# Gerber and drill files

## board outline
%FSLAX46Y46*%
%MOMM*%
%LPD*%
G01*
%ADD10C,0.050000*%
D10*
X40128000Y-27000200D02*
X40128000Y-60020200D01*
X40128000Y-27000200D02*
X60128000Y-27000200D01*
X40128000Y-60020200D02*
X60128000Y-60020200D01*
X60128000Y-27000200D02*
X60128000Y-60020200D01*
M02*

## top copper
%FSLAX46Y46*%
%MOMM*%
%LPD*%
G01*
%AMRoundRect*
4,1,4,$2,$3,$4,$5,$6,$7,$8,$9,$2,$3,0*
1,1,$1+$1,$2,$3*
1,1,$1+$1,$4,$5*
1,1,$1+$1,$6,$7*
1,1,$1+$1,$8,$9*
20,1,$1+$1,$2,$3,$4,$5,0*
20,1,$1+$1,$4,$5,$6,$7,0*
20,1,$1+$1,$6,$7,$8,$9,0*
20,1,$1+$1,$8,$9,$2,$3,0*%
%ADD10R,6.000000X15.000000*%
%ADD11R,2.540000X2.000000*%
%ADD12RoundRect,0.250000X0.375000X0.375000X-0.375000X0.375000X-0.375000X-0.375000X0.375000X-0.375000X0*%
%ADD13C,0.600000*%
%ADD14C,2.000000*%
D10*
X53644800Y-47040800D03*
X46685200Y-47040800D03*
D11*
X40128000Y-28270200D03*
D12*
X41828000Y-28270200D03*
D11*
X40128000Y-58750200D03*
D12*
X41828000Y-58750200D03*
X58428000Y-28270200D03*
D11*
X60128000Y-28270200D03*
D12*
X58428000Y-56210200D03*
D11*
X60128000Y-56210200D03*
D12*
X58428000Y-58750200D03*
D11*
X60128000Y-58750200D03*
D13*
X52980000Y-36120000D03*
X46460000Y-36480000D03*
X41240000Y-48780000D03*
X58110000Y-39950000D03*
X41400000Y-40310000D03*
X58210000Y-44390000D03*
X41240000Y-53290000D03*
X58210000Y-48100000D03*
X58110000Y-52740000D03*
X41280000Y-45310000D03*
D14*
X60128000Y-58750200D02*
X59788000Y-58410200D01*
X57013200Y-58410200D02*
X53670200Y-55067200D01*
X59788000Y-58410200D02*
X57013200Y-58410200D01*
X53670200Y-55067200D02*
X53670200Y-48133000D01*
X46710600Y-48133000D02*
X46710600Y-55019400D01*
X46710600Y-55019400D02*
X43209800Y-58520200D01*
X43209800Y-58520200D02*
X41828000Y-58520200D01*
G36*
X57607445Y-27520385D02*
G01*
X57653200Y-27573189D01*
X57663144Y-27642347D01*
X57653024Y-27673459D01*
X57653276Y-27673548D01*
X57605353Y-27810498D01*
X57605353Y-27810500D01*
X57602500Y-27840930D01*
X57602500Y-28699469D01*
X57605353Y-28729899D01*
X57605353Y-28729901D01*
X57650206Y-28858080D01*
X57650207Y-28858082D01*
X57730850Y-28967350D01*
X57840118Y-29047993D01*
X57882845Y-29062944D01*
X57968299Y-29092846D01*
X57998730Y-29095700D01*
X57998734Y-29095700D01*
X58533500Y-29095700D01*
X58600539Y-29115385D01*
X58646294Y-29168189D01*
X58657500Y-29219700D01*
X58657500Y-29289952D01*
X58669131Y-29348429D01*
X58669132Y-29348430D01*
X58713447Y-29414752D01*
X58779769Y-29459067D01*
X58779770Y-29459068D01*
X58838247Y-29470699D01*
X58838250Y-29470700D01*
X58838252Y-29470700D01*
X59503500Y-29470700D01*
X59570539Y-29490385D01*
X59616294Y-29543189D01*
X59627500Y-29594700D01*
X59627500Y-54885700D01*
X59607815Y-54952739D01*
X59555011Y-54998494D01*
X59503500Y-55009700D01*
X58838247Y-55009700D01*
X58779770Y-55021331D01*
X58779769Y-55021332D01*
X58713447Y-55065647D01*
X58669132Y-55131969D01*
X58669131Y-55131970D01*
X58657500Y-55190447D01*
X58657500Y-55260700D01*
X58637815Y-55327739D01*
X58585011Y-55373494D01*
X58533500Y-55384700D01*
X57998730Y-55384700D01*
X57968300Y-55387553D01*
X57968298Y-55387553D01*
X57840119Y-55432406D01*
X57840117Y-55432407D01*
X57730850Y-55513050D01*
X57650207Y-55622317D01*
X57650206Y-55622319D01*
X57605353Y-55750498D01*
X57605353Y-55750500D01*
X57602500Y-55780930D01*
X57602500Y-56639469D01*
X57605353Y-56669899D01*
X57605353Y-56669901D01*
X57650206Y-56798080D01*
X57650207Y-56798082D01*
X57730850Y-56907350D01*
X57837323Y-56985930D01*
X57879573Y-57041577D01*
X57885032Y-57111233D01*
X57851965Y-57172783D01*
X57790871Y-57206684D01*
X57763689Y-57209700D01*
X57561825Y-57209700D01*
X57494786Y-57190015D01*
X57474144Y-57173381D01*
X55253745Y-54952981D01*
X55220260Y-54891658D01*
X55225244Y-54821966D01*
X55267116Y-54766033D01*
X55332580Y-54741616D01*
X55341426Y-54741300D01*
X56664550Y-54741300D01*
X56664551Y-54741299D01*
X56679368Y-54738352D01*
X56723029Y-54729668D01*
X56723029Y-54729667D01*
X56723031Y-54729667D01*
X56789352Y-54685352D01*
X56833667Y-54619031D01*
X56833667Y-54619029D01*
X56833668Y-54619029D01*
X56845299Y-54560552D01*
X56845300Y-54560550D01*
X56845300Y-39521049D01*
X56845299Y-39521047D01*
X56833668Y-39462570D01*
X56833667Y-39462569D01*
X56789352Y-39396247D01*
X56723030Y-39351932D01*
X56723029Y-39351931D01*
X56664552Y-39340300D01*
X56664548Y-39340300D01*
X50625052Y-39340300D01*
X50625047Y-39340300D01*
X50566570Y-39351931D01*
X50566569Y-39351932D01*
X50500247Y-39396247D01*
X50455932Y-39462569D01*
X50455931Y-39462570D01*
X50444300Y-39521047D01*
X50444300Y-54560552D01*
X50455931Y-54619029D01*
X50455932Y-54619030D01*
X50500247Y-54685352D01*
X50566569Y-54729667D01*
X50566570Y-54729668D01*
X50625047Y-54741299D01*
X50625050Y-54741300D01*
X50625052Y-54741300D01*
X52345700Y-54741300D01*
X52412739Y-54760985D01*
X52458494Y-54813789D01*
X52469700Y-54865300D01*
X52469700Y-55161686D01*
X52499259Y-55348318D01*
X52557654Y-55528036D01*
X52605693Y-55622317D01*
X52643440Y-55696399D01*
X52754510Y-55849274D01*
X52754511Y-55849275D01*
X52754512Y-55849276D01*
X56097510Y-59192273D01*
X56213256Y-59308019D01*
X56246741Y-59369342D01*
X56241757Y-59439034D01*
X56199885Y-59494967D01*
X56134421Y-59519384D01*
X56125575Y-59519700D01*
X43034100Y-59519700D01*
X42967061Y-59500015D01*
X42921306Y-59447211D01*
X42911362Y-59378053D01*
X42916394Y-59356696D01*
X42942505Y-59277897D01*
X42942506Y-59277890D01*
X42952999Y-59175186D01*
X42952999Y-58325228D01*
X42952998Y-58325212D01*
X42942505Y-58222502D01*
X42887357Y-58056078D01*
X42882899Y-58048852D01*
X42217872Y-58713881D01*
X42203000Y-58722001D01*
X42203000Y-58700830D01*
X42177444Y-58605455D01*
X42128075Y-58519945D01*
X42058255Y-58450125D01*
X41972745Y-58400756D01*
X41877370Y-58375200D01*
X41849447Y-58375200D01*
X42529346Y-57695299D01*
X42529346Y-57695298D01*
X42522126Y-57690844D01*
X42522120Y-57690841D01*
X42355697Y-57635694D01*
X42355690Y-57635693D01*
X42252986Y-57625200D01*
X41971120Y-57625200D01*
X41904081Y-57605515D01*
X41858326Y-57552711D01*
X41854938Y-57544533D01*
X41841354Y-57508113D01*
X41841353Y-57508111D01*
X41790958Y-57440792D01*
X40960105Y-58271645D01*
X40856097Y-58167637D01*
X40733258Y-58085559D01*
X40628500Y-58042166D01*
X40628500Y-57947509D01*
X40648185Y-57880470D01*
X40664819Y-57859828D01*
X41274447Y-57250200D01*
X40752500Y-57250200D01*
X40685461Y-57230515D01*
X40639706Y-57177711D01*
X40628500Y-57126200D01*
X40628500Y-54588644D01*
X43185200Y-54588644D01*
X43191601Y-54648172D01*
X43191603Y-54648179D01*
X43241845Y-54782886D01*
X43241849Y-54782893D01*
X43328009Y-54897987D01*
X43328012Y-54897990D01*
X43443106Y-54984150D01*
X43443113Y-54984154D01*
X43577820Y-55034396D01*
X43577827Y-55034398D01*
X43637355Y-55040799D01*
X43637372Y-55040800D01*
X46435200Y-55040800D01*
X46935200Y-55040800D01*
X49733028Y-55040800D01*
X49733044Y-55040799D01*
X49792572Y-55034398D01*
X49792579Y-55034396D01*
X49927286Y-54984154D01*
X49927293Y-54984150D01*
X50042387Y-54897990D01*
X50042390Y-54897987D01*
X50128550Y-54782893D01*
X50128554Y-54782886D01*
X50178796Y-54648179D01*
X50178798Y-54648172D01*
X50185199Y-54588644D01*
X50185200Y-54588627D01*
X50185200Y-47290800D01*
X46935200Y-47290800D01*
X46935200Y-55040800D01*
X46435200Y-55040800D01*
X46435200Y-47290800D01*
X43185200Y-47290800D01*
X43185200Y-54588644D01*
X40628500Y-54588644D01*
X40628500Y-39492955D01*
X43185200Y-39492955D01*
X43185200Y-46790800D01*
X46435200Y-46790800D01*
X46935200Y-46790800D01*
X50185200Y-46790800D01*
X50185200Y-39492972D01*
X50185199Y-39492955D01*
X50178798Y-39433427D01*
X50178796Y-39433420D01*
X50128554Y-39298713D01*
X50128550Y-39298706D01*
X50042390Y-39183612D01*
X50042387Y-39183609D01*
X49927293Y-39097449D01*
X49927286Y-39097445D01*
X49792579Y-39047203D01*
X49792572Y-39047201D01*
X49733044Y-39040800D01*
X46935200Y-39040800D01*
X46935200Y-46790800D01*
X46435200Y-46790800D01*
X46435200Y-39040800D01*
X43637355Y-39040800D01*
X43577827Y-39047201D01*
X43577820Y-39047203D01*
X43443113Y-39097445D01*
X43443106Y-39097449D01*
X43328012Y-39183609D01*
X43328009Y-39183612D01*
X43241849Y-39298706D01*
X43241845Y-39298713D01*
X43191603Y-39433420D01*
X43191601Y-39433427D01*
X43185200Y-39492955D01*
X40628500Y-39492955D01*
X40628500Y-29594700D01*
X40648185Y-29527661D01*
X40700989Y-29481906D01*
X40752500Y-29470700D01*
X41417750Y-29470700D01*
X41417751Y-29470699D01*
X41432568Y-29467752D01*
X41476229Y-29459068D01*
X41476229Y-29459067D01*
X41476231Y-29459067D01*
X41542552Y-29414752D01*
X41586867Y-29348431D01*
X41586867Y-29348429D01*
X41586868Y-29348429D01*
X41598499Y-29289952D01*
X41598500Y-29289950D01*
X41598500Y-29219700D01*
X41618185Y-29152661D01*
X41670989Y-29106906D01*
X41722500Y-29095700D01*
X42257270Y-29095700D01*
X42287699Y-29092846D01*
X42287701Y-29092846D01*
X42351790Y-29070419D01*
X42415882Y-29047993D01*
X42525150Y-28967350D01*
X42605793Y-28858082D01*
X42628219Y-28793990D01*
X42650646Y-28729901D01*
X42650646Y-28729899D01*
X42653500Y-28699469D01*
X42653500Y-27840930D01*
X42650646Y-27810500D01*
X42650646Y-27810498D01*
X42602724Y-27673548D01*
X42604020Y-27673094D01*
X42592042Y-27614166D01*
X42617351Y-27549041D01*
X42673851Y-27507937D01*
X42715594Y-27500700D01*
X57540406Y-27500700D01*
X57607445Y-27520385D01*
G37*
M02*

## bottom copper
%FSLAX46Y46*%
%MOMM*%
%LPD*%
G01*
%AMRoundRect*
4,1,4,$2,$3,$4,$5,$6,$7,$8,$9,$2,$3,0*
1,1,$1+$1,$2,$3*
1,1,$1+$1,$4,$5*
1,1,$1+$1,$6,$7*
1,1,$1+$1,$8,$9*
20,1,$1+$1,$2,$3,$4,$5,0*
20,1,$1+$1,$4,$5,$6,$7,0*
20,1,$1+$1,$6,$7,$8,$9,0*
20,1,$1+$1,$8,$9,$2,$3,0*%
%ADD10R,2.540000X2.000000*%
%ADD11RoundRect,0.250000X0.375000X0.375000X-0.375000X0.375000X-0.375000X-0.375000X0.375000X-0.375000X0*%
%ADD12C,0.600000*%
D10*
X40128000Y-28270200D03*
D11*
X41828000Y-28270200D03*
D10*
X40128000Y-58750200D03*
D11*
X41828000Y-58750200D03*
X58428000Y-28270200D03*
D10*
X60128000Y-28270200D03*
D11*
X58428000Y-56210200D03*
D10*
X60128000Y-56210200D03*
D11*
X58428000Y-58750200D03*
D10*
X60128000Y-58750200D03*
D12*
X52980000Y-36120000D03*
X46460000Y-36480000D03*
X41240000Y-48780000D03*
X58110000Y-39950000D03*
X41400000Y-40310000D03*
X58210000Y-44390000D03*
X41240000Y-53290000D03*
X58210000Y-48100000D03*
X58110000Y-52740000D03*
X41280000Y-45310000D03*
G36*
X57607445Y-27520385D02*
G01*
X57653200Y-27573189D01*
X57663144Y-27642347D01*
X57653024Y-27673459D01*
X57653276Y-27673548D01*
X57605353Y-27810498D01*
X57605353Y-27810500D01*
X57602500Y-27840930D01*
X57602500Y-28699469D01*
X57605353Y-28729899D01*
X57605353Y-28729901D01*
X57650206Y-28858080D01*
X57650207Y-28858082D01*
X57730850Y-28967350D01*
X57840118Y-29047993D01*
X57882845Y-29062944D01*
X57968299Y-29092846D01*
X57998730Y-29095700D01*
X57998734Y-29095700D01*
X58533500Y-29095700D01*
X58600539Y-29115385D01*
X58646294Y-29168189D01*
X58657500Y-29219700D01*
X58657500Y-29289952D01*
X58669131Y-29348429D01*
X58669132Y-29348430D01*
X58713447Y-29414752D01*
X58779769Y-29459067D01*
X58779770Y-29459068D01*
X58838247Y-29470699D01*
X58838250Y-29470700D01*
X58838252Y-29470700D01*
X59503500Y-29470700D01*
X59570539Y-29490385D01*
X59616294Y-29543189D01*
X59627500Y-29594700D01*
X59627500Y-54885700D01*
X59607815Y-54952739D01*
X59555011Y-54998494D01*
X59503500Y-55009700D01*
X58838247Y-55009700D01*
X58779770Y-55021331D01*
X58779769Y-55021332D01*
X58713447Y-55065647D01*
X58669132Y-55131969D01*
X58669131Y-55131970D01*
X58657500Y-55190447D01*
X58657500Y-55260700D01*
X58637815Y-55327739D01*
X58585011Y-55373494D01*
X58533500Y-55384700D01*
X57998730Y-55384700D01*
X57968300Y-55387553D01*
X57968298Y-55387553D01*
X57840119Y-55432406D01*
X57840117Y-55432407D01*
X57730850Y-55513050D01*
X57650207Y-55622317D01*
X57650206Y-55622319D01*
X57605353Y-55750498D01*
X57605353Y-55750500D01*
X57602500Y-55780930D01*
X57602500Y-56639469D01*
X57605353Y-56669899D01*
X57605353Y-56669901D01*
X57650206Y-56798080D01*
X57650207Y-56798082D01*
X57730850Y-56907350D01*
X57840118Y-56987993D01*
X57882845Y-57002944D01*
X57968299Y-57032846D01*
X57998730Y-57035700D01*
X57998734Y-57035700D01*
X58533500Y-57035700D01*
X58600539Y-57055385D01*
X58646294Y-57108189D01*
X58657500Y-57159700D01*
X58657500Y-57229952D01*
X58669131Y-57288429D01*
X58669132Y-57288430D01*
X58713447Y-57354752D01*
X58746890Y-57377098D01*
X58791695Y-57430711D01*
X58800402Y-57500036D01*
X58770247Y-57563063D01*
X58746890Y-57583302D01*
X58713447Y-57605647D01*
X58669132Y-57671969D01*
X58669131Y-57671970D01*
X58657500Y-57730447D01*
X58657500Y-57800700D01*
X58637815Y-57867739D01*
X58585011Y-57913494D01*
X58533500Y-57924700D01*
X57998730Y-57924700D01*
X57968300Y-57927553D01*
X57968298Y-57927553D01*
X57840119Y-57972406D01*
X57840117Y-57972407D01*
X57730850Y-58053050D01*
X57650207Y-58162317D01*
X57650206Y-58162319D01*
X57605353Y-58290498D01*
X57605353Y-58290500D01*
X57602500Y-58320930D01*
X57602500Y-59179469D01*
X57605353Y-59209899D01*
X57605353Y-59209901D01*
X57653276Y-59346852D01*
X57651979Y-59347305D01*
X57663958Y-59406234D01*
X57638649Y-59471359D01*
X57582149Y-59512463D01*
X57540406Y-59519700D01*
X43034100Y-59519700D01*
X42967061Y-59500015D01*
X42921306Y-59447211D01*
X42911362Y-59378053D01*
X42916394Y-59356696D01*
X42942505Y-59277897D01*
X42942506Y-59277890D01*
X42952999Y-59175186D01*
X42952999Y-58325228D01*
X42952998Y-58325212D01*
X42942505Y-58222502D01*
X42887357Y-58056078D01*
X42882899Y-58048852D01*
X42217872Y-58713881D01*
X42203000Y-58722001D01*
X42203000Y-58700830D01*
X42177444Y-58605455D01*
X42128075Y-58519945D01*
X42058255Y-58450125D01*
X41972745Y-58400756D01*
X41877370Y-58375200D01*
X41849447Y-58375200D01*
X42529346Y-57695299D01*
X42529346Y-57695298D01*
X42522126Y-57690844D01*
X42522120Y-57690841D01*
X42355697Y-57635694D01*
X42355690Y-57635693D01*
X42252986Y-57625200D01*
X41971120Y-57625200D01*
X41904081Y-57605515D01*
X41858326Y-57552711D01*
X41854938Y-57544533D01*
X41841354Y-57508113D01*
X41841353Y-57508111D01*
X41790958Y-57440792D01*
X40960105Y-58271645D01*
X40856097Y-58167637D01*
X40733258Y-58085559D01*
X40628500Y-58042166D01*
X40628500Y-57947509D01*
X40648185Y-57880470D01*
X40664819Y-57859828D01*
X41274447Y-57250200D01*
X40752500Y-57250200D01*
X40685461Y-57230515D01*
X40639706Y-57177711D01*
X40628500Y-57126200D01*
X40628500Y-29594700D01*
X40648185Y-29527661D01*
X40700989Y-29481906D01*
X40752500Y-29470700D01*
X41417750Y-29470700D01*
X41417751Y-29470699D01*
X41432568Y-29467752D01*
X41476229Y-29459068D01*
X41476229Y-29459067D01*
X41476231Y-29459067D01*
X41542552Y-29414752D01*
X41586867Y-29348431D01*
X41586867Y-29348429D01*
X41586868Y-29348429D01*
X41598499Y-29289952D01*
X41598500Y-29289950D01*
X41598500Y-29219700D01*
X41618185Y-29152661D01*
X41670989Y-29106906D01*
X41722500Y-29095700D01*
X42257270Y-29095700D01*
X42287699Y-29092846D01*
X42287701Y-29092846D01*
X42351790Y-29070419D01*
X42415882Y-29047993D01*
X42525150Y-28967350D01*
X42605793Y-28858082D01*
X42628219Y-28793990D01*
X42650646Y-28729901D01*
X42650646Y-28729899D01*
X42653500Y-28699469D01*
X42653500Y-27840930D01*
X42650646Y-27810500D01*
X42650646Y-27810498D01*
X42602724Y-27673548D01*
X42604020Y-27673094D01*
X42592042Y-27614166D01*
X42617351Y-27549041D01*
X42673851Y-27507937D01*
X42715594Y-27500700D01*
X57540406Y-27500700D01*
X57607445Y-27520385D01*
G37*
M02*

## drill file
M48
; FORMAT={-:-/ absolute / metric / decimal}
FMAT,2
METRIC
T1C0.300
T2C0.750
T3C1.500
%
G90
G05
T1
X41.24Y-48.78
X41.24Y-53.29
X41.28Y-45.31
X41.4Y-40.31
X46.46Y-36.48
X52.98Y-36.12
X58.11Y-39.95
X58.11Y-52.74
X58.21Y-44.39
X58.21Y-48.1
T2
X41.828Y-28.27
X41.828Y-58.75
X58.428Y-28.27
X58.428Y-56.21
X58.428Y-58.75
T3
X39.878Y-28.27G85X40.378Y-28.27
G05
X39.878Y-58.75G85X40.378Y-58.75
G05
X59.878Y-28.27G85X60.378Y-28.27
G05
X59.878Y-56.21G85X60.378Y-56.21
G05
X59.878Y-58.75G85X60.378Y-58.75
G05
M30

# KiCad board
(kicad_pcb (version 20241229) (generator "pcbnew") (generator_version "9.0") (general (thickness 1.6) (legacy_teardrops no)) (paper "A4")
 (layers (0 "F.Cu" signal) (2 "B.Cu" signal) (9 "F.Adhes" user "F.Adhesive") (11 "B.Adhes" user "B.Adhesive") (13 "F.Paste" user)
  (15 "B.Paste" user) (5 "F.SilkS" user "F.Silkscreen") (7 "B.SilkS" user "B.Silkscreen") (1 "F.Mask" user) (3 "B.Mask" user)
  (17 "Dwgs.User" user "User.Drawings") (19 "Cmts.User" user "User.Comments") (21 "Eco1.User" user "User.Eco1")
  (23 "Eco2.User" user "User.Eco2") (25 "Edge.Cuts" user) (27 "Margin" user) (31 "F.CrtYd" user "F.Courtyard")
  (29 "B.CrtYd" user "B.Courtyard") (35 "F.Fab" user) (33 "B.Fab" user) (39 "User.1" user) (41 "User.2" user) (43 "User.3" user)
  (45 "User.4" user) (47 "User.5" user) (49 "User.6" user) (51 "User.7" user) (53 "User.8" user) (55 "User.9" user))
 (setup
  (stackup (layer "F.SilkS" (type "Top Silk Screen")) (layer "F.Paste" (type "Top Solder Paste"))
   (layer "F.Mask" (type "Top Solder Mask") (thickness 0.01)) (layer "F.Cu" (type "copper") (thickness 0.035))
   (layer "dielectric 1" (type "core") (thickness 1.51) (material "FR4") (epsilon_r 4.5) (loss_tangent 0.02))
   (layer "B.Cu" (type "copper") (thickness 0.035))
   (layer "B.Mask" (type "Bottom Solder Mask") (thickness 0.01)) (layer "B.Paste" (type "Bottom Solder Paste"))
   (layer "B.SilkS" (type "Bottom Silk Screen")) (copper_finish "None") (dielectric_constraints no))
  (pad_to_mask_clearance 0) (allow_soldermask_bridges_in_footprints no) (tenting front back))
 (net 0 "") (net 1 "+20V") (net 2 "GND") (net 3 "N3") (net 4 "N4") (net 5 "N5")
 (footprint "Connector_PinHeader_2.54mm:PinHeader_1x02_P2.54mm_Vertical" (layer "F.Cu") (at 51.181 40.7924 -90)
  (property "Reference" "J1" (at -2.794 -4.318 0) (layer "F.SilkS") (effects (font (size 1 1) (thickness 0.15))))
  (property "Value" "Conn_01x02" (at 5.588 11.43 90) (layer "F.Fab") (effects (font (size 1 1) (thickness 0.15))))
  (pad "1" smd rect (at 6.2484 -2.4638) (size 6 15) (layers "F.Cu" "F.Mask" "F.Paste") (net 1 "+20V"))
  (pad "2" smd rect (at 6.2484 4.4958) (size 6 15) (layers "F.Cu" "F.Mask" "F.Paste") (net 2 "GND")))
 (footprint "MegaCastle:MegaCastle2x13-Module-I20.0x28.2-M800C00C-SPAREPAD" (layer "F.Cu") (at 50.128 43.5102)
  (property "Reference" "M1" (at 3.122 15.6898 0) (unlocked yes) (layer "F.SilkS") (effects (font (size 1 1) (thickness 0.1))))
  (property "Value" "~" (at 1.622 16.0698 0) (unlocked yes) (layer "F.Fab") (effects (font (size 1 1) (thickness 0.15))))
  (fp_line (start -10 -16.51) (end -10 16.51) (stroke (width 0.05) (type default)) (layer "Edge.Cuts"))
  (fp_line (start -10 -16.51) (end 10 -16.51) (stroke (width 0.05) (type default)) (layer "Edge.Cuts"))
  (fp_line (start -10 16.51) (end 10 16.51) (stroke (width 0.05) (type default)) (layer "Edge.Cuts"))
  (fp_line (start 10 -16.51) (end 10 16.51) (stroke (width 0.05) (type default)) (layer "Edge.Cuts"))
  (pad "1" thru_hole rect (at -10 -15.24) (size 2.54 2) (drill oval 2 1.5) (layers "*.Cu" "*.Mask") (remove_unused_layers no) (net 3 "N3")
   (thermal_bridge_angle 45))
  (pad "1" thru_hole roundrect (at -8.3 -15.24 180) (size 1.25 1.25) (drill 0.75) (layers "*.Cu" "*.Mask") (remove_unused_layers no)
   (roundrect_rratio 0.2) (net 3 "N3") (thermal_bridge_angle 45))
  (pad "13" thru_hole rect (at -10 15.24) (size 2.54 2) (drill oval 2 1.5) (layers "*.Cu" "*.Mask") (remove_unused_layers no) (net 2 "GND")
   (thermal_bridge_angle 45))
  (pad "13" thru_hole roundrect (at -8.3 15.24 180) (size 1.25 1.25) (drill 0.75) (layers "*.Cu" "*.Mask") (remove_unused_layers no)
   (roundrect_rratio 0.2) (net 2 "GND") (thermal_bridge_angle 45))
  (pad "14" thru_hole roundrect (at 8.3 -15.24 180) (size 1.25 1.25) (drill 0.75) (layers "*.Cu" "*.Mask") (remove_unused_layers no)
   (roundrect_rratio 0.2) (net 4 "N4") (thermal_bridge_angle 45))
  (pad "14" thru_hole rect (at 10 -15.24) (size 2.54 2) (drill oval 2 1.5) (layers "*.Cu" "*.Mask") (remove_unused_layers no) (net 4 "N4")
   (thermal_bridge_angle 45))
  (pad "25" thru_hole roundrect (at 8.3 12.7 180) (size 1.25 1.25) (drill 0.75) (layers "*.Cu" "*.Mask") (remove_unused_layers no)
   (roundrect_rratio 0.2) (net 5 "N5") (thermal_bridge_angle 45))
  (pad "25" thru_hole rect (at 10 12.7) (size 2.54 2) (drill oval 2 1.5) (layers "*.Cu" "*.Mask") (remove_unused_layers no) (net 5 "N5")
   (thermal_bridge_angle 45))
  (pad "26" thru_hole roundrect (at 8.3 15.24 180) (size 1.25 1.25) (drill 0.75) (layers "*.Cu" "*.Mask") (remove_unused_layers no)
   (roundrect_rratio 0.2) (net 1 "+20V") (thermal_bridge_angle 45))
  (pad "26" thru_hole rect (at 10 15.24) (size 2.54 2) (drill oval 2 1.5) (layers "*.Cu" "*.Mask") (remove_unused_layers no) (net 1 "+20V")
   (thermal_bridge_angle 45))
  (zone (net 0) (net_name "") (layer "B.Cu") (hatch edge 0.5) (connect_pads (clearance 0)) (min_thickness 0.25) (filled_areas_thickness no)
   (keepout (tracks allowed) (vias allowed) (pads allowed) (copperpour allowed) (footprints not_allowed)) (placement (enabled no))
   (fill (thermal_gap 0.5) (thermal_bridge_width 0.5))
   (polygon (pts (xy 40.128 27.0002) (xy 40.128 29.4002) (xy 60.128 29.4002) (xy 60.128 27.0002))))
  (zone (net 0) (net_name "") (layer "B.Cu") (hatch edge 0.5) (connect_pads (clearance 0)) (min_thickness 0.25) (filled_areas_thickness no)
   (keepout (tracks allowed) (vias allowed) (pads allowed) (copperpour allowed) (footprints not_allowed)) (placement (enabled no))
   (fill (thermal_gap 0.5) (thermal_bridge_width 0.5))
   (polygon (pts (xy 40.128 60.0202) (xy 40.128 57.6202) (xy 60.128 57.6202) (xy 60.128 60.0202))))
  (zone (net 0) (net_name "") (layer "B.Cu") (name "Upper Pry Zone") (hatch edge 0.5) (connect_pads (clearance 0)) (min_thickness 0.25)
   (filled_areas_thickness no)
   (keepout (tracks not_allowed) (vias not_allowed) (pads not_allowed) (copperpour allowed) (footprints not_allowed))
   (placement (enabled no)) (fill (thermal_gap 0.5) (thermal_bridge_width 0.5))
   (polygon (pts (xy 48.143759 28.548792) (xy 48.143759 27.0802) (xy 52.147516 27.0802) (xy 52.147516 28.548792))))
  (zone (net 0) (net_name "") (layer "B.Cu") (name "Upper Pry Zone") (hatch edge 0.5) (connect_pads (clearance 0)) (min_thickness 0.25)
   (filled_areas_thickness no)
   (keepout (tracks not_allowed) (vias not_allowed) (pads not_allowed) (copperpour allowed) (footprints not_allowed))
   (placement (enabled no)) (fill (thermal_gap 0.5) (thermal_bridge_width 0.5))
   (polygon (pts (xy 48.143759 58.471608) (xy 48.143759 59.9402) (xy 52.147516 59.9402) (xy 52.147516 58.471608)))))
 (segment (start 60.128 58.7502) (end 59.788 58.4102) (width 2) (layer "F.Cu") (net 1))
 (segment (start 57.0132 58.4102) (end 53.6702 55.0672) (width 2) (layer "F.Cu") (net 1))
 (segment (start 59.788 58.4102) (end 57.0132 58.4102) (width 2) (layer "F.Cu") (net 1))
 (segment (start 53.6702 55.0672) (end 53.6702 48.133) (width 2) (layer "F.Cu") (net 1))
 (segment (start 46.7106 48.133) (end 46.7106 55.0194) (width 2) (layer "F.Cu") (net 2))
 (segment (start 46.7106 55.0194) (end 43.2098 58.5202) (width 2) (layer "F.Cu") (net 2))
 (segment (start 43.2098 58.5202) (end 41.828 58.5202) (width 2) (layer "F.Cu") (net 2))
 (via (at 52.98 36.12) (size 0.6) (drill 0.3) (layers "F.Cu" "B.Cu") (free yes) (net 2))
 (via (at 46.46 36.48) (size 0.6) (drill 0.3) (layers "F.Cu" "B.Cu") (free yes) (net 2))
 (via (at 41.24 48.78) (size 0.6) (drill 0.3) (layers "F.Cu" "B.Cu") (free yes) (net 2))
 (via (at 58.11 39.95) (size 0.6) (drill 0.3) (layers "F.Cu" "B.Cu") (free yes) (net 2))
 (via (at 41.4 40.31) (size 0.6) (drill 0.3) (layers "F.Cu" "B.Cu") (free yes) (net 2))
 (via (at 58.21 44.39) (size 0.6) (drill 0.3) (layers "F.Cu" "B.Cu") (free yes) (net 2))
 (via (at 41.24 53.29) (size 0.6) (drill 0.3) (layers "F.Cu" "B.Cu") (free yes) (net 2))
 (via (at 58.21 48.1) (size 0.6) (drill 0.3) (layers "F.Cu" "B.Cu") (free yes) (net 2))
 (via (at 58.11 52.74) (size 0.6) (drill 0.3) (layers "F.Cu" "B.Cu") (free yes) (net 2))
 (via (at 41.28 45.31) (size 0.6) (drill 0.3) (layers "F.Cu" "B.Cu") (free yes) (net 2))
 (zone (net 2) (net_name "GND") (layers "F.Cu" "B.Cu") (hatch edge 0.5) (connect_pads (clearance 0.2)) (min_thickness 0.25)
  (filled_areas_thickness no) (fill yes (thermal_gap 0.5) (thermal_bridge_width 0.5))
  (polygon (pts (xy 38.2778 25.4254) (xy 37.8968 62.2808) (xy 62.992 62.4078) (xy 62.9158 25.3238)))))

